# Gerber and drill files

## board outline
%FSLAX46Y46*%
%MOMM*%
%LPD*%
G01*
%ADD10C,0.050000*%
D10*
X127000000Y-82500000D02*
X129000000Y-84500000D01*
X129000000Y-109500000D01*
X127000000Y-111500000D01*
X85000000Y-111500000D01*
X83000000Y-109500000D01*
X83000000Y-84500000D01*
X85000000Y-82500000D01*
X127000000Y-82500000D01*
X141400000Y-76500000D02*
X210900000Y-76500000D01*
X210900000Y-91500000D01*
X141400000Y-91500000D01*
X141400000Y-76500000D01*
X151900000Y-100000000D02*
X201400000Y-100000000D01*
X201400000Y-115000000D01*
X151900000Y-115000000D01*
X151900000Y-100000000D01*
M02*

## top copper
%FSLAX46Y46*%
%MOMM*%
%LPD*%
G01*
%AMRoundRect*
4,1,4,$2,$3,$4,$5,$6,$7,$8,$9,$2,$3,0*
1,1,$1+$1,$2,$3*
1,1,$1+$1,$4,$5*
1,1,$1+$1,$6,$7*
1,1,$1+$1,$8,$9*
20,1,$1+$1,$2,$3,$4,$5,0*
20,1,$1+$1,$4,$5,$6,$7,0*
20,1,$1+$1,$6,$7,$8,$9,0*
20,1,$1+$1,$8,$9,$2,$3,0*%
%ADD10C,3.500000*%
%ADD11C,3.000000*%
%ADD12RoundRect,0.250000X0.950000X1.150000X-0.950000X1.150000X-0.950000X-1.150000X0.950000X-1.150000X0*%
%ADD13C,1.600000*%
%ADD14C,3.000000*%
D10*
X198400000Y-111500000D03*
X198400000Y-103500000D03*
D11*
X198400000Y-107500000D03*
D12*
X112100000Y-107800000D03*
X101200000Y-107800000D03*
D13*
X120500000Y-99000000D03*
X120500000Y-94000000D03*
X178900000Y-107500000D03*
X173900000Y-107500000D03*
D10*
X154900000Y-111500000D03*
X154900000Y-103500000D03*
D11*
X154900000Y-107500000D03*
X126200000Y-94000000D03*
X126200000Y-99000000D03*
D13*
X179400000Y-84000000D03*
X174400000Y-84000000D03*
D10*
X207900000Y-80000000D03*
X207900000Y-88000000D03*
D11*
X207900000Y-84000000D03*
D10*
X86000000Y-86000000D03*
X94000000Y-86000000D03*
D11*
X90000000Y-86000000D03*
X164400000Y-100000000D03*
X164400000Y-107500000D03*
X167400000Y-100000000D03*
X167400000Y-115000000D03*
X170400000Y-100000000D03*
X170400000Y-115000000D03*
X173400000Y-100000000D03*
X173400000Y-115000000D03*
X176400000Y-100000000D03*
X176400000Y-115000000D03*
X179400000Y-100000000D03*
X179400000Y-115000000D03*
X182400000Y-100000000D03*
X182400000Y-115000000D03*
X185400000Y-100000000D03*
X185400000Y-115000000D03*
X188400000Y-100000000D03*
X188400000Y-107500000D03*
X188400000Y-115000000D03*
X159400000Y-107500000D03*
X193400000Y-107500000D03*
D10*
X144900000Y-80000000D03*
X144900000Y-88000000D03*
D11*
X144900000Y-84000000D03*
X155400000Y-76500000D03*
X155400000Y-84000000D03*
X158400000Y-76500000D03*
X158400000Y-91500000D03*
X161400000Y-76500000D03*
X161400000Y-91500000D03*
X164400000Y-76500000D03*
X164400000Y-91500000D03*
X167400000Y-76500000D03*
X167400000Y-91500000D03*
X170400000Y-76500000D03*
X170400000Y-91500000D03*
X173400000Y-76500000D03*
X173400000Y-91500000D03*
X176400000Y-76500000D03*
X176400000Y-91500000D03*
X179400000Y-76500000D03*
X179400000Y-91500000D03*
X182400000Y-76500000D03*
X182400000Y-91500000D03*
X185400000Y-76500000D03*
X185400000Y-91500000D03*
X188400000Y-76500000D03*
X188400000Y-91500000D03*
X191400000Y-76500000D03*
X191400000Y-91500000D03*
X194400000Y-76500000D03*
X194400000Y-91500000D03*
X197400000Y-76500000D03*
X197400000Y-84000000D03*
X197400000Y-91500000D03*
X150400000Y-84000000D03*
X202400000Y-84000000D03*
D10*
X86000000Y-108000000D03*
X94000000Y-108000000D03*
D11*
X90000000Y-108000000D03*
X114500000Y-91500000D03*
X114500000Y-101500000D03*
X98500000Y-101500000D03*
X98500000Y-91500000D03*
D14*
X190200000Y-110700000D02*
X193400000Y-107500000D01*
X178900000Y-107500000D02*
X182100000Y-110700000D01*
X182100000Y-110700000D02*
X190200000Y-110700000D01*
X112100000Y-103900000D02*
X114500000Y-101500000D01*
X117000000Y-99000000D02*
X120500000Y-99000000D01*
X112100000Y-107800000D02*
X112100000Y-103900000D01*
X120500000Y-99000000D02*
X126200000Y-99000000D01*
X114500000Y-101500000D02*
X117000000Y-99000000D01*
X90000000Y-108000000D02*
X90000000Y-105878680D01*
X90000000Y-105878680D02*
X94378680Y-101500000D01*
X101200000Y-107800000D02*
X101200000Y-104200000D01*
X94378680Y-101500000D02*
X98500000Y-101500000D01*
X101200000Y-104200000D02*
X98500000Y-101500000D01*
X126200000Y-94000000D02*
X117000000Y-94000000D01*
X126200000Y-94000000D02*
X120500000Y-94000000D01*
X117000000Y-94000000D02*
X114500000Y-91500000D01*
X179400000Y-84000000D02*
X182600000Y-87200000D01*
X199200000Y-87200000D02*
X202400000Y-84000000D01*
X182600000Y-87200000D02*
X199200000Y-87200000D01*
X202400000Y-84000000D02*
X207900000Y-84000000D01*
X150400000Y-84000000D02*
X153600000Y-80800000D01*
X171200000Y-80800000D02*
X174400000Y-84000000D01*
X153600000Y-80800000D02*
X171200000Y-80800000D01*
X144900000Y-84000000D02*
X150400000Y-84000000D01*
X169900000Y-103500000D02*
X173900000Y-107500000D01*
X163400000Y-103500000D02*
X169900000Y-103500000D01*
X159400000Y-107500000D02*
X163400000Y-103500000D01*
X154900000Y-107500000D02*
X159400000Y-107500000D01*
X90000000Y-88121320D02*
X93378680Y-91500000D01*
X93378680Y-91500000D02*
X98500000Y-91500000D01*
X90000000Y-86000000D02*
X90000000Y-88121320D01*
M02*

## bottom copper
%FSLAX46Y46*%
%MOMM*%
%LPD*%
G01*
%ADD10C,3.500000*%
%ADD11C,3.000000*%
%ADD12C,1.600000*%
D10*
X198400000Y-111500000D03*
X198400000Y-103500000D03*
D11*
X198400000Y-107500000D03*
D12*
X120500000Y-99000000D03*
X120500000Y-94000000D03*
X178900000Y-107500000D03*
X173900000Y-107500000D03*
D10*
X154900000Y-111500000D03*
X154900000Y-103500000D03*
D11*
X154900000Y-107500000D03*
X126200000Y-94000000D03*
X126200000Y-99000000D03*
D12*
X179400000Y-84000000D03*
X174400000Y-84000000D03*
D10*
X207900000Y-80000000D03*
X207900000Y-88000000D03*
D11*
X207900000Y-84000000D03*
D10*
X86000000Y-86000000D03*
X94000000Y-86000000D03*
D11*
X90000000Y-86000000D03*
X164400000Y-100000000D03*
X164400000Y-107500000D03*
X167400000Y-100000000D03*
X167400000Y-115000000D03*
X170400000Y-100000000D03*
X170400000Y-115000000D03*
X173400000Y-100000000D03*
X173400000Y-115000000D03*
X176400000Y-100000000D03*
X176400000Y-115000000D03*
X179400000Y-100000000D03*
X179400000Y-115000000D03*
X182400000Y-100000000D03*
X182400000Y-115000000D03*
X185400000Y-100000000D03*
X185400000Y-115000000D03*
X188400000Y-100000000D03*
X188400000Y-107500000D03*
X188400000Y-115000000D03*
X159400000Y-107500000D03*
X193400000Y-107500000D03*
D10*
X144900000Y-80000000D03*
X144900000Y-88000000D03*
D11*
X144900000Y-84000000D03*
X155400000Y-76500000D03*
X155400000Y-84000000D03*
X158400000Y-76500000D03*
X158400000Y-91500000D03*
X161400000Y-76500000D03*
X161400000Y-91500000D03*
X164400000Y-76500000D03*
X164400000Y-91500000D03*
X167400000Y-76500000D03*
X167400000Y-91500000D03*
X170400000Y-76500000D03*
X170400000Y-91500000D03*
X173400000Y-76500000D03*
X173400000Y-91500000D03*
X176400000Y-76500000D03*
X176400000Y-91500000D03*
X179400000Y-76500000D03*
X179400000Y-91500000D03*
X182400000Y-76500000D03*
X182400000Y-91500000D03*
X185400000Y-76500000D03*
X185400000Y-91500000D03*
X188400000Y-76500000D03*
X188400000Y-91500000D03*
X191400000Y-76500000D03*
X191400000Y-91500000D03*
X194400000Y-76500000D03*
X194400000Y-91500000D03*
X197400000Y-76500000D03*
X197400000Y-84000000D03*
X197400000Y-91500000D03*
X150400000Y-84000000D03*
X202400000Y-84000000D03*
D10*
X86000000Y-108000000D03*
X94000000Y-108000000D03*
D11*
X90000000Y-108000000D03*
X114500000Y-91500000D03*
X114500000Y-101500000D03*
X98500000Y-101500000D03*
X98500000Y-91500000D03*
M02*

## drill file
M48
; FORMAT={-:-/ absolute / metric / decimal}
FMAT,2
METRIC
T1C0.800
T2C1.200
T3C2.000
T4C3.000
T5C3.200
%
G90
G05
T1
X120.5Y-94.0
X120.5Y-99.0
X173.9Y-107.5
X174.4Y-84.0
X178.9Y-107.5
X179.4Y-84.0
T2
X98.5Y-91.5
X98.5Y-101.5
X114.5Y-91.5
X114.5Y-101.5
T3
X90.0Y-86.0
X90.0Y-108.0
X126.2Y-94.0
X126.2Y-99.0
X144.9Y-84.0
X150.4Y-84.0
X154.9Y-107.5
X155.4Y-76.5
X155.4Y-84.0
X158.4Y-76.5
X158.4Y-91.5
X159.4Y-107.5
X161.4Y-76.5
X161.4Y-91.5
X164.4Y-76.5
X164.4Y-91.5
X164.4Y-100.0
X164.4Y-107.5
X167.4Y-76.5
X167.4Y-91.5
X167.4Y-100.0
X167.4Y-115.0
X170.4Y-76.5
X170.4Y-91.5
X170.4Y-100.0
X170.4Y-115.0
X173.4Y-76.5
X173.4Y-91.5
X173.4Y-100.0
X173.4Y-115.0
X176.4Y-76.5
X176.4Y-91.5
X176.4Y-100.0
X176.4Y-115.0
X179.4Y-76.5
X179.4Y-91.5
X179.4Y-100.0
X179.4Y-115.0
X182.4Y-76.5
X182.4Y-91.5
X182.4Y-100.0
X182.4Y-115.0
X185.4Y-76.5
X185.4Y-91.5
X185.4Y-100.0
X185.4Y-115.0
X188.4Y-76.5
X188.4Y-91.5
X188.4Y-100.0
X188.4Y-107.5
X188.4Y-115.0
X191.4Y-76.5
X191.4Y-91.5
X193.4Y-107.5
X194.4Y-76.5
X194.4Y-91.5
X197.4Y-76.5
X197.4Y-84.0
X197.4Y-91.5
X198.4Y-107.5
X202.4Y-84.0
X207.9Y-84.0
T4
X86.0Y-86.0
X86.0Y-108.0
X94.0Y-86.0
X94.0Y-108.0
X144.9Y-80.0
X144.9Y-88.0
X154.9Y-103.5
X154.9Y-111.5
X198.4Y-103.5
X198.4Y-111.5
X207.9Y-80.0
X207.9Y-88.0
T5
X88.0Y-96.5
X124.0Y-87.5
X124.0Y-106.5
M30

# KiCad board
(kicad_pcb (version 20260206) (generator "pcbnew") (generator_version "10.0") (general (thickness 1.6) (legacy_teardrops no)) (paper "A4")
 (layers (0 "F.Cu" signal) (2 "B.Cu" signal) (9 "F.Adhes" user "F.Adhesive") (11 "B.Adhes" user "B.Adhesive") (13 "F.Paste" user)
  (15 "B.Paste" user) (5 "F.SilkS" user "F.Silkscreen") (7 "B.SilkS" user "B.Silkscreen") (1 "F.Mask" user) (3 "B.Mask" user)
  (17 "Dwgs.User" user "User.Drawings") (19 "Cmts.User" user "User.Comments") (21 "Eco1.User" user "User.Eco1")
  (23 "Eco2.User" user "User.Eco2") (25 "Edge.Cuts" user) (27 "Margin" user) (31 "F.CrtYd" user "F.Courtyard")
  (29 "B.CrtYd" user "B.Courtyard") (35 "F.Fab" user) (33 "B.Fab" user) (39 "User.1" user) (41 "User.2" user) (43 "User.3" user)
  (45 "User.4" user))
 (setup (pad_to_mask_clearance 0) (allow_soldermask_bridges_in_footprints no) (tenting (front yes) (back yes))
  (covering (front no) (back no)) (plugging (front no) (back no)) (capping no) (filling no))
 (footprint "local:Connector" (layer "F.Cu") (at 198.4 107.5 180)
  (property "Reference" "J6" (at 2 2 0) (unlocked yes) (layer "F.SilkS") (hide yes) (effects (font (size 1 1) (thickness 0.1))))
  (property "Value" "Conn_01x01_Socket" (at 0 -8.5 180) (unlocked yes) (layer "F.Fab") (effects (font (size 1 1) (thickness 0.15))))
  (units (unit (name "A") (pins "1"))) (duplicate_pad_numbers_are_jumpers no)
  (pad "" thru_hole circle (at 0 -4 190) (size 3.5 3.5) (drill 3) (layers "*.Cu" "*.Mask") (remove_unused_layers no))
  (pad "" thru_hole circle (at 0 4 190) (size 3.5 3.5) (drill 3) (layers "*.Cu" "*.Mask") (remove_unused_layers no))
  (pad "1" thru_hole circle (at 0 0 190) (size 3 3) (drill 2) (layers "*.Cu" "*.Mask") (remove_unused_layers no) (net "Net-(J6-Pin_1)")))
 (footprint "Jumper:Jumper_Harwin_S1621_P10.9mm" (layer "F.Cu") (at 106.65 107.8 180)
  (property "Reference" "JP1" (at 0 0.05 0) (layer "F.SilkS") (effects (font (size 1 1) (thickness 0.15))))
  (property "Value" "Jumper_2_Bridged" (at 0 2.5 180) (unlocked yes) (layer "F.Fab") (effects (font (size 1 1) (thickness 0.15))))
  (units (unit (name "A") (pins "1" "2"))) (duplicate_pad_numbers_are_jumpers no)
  (pad "1" smd roundrect (at -5.45 0 180) (size 2.4 2.8) (layers "F.Cu" "F.Mask" "F.Paste") (roundrect_rratio 0.1041666667)
   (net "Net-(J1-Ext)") (thermal_bridge_angle 45))
  (pad "2" smd roundrect (at 5.45 0 180) (size 2.4 2.8) (layers "F.Cu" "F.Mask" "F.Paste") (roundrect_rratio 0.1041666667)
   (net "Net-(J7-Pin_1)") (thermal_bridge_angle 45)))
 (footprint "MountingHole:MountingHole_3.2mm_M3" (layer "F.Cu") (at 124 106.5)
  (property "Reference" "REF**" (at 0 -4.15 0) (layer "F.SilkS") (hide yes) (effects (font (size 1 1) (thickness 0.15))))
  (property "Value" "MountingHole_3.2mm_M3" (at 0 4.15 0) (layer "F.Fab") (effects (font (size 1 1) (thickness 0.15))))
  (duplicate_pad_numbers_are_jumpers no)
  (pad "" np_thru_hole circle (at 0 0) (size 3.2 3.2) (drill 3.2) (layers "*.Cu" "*.Mask")))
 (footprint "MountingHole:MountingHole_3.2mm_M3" (layer "F.Cu") (at 88 96.5)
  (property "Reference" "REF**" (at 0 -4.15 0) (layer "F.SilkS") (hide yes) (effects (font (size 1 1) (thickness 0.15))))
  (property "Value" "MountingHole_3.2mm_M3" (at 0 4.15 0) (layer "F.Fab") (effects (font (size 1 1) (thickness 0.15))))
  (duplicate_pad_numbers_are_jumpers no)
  (pad "" np_thru_hole circle (at 0 0) (size 3.2 3.2) (drill 3.2) (layers "*.Cu" "*.Mask")))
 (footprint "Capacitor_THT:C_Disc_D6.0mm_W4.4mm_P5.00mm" (layer "F.Cu") (at 120.5 99 90)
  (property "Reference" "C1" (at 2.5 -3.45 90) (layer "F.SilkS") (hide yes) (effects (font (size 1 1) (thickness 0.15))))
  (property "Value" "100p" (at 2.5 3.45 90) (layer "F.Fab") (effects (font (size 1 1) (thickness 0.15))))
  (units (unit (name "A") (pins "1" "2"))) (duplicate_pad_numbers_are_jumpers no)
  (pad "1" thru_hole circle (at 0 0 90) (size 1.6 1.6) (drill 0.8) (layers "*.Cu" "*.Mask") (remove_unused_layers no) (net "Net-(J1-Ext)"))
  (pad "2" thru_hole circle (at 5 0 90) (size 1.6 1.6) (drill 0.8) (layers "*.Cu" "*.Mask") (remove_unused_layers no) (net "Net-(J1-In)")))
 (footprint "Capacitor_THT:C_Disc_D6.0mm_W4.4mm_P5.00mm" (layer "F.Cu") (at 178.9 107.5 180)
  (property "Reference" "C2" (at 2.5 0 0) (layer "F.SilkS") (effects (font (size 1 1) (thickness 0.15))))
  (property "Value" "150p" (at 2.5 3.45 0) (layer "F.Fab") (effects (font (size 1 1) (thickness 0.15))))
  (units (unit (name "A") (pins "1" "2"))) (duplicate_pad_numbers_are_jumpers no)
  (pad "1" thru_hole circle (at 0 0 180) (size 1.6 1.6) (drill 0.8) (layers "*.Cu" "*.Mask") (remove_unused_layers no)
   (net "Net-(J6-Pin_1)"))
  (pad "2" thru_hole circle (at 5 0 180) (size 1.6 1.6) (drill 0.8) (layers "*.Cu" "*.Mask") (remove_unused_layers no)
   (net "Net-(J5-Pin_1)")))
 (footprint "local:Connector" (layer "F.Cu") (at 154.9 107.5 180)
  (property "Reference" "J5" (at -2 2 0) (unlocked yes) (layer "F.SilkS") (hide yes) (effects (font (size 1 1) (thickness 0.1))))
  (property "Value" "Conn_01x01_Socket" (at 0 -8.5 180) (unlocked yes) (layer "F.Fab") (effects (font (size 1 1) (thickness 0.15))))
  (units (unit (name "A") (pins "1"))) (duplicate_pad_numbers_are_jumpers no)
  (pad "" thru_hole circle (at 0 -4 190) (size 3.5 3.5) (drill 3) (layers "*.Cu" "*.Mask") (remove_unused_layers no))
  (pad "" thru_hole circle (at 0 4 190) (size 3.5 3.5) (drill 3) (layers "*.Cu" "*.Mask") (remove_unused_layers no))
  (pad "1" thru_hole circle (at 0 0 190) (size 3 3) (drill 2) (layers "*.Cu" "*.Mask") (remove_unused_layers no) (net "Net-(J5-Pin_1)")))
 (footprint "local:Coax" (layer "F.Cu") (at 126.2 96)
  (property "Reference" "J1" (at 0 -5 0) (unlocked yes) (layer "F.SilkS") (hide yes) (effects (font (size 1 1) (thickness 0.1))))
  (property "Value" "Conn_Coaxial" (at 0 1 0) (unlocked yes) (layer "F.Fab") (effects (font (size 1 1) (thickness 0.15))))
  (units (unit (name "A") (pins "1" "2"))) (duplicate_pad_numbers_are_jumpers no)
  (pad "1" thru_hole circle (at 0 -2 10) (size 3 3) (drill 2) (layers "*.Cu" "*.Mask") (remove_unused_layers no) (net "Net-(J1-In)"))
  (pad "2" thru_hole circle (at 0 3 10) (size 3 3) (drill 2) (layers "*.Cu" "*.Mask") (remove_unused_layers no) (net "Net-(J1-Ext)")))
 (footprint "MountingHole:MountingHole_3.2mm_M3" (layer "F.Cu") (at 124 87.5)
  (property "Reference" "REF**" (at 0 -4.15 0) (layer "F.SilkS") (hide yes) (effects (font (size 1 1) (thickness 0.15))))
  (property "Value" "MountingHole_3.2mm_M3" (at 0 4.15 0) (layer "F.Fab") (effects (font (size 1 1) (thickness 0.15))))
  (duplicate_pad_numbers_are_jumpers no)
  (pad "" np_thru_hole circle (at 0 0) (size 3.2 3.2) (drill 3.2) (layers "*.Cu" "*.Mask")))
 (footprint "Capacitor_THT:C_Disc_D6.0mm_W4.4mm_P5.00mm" (layer "F.Cu") (at 179.4 84 180)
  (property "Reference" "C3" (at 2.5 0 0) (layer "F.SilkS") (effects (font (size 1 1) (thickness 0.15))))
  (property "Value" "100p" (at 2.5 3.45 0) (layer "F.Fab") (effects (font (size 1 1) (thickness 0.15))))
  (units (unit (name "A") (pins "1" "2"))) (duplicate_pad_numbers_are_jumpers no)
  (pad "1" thru_hole circle (at 0 0 180) (size 1.6 1.6) (drill 0.8) (layers "*.Cu" "*.Mask") (remove_unused_layers no)
   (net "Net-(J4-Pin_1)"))
  (pad "2" thru_hole circle (at 5 0 180) (size 1.6 1.6) (drill 0.8) (layers "*.Cu" "*.Mask") (remove_unused_layers no)
   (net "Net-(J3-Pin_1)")))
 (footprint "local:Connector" (layer "F.Cu") (at 207.9 84)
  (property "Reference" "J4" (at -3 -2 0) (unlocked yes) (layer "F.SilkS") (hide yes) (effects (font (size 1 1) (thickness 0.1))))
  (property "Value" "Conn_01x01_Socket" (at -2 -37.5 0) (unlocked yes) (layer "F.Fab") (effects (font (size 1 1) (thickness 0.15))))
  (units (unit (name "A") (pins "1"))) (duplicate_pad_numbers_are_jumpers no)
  (pad "" thru_hole circle (at 0 -4 10) (size 3.5 3.5) (drill 3) (layers "*.Cu" "*.Mask") (remove_unused_layers no))
  (pad "" thru_hole circle (at 0 4 10) (size 3.5 3.5) (drill 3) (layers "*.Cu" "*.Mask") (remove_unused_layers no))
  (pad "1" thru_hole circle (at 0 0 10) (size 3 3) (drill 2) (layers "*.Cu" "*.Mask") (remove_unused_layers no) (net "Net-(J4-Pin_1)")))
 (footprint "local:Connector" (layer "F.Cu") (at 90 86 90)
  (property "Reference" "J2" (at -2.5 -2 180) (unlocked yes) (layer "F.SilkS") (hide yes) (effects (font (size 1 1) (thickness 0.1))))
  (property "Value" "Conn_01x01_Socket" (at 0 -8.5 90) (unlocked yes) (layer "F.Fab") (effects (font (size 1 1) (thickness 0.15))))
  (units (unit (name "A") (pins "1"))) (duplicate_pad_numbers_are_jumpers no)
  (pad "" thru_hole circle (at 0 -4 100) (size 3.5 3.5) (drill 3) (layers "*.Cu" "*.Mask") (remove_unused_layers no))
  (pad "" thru_hole circle (at 0 4 100) (size 3.5 3.5) (drill 3) (layers "*.Cu" "*.Mask") (remove_unused_layers no))
  (pad "1" thru_hole circle (at 0 0 100) (size 3 3) (drill 2) (layers "*.Cu" "*.Mask") (remove_unused_layers no) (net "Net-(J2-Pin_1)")))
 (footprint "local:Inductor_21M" (layer "F.Cu") (at 167.4 107)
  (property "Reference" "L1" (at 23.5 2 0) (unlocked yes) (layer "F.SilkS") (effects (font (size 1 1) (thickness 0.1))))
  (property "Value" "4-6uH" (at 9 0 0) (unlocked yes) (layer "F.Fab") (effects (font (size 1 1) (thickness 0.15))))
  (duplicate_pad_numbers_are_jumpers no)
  (pad "" thru_hole circle (at -3 -7 10) (size 3 3) (drill 2) (layers "*.Cu" "*.Mask") (remove_unused_layers no))
  (pad "" thru_hole circle (at -3 0.5 10) (size 3 3) (drill 2) (layers "*.Cu" "*.Mask") (remove_unused_layers no))
  (pad "" thru_hole circle (at 0 -7 10) (size 3 3) (drill 2) (layers "*.Cu" "*.Mask") (remove_unused_layers no))
  (pad "" thru_hole circle (at 0 8 10) (size 3 3) (drill 2) (layers "*.Cu" "*.Mask") (remove_unused_layers no))
  (pad "" thru_hole circle (at 3 -7 10) (size 3 3) (drill 2) (layers "*.Cu" "*.Mask") (remove_unused_layers no))
  (pad "" thru_hole circle (at 3 8 10) (size 3 3) (drill 2) (layers "*.Cu" "*.Mask") (remove_unused_layers no))
  (pad "" thru_hole circle (at 6 -7 10) (size 3 3) (drill 2) (layers "*.Cu" "*.Mask") (remove_unused_layers no))
  (pad "" thru_hole circle (at 6 8 10) (size 3 3) (drill 2) (layers "*.Cu" "*.Mask") (remove_unused_layers no))
  (pad "" thru_hole circle (at 9 -7 10) (size 3 3) (drill 2) (layers "*.Cu" "*.Mask") (remove_unused_layers no))
  (pad "" thru_hole circle (at 9 8 10) (size 3 3) (drill 2) (layers "*.Cu" "*.Mask") (remove_unused_layers no))
  (pad "" thru_hole circle (at 12 -7 10) (size 3 3) (drill 2) (layers "*.Cu" "*.Mask") (remove_unused_layers no))
  (pad "" thru_hole circle (at 12 8 10) (size 3 3) (drill 2) (layers "*.Cu" "*.Mask") (remove_unused_layers no))
  (pad "" thru_hole circle (at 15 -7 10) (size 3 3) (drill 2) (layers "*.Cu" "*.Mask") (remove_unused_layers no))
  (pad "" thru_hole circle (at 15 8 10) (size 3 3) (drill 2) (layers "*.Cu" "*.Mask") (remove_unused_layers no))
  (pad "" thru_hole circle (at 18 -7 10) (size 3 3) (drill 2) (layers "*.Cu" "*.Mask") (remove_unused_layers no))
  (pad "" thru_hole circle (at 18 8 10) (size 3 3) (drill 2) (layers "*.Cu" "*.Mask") (remove_unused_layers no))
  (pad "" thru_hole circle (at 21 -7 10) (size 3 3) (drill 2) (layers "*.Cu" "*.Mask") (remove_unused_layers no))
  (pad "" thru_hole circle (at 21 0.5 10) (size 3 3) (drill 2) (layers "*.Cu" "*.Mask") (remove_unused_layers no))
  (pad "" thru_hole circle (at 21 8 10) (size 3 3) (drill 2) (layers "*.Cu" "*.Mask") (remove_unused_layers no))
  (pad "1" thru_hole circle (at -8 0.5 10) (size 3 3) (drill 2) (layers "*.Cu" "*.Mask") (remove_unused_layers no) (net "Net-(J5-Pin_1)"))
  (pad "2" thru_hole circle (at 26 0.5 10) (size 3 3) (drill 2) (layers "*.Cu" "*.Mask") (remove_unused_layers no) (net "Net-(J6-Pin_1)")))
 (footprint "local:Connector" (layer "F.Cu") (at 144.9 84)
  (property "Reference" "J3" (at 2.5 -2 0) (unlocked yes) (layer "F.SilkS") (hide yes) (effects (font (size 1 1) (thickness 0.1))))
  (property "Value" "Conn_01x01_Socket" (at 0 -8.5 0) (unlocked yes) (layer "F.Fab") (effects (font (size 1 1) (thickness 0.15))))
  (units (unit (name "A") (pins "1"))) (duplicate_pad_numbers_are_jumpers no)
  (pad "" thru_hole circle (at 0 -4 10) (size 3.5 3.5) (drill 3) (layers "*.Cu" "*.Mask") (remove_unused_layers no))
  (pad "" thru_hole circle (at 0 4 10) (size 3.5 3.5) (drill 3) (layers "*.Cu" "*.Mask") (remove_unused_layers no))
  (pad "1" thru_hole circle (at 0 0 10) (size 3 3) (drill 2) (layers "*.Cu" "*.Mask") (remove_unused_layers no) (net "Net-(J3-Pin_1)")))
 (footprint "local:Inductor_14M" (layer "F.Cu") (at 176.4 83.5)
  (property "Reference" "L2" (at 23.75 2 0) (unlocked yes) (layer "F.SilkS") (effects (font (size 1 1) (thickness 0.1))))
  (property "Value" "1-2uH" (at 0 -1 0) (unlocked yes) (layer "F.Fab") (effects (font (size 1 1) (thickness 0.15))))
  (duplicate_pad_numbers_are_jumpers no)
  (pad "" thru_hole circle (at -21 -7 10) (size 3 3) (drill 2) (layers "*.Cu" "*.Mask") (remove_unused_layers no))
  (pad "" thru_hole circle (at -21 0.5 10) (size 3 3) (drill 2) (layers "*.Cu" "*.Mask") (remove_unused_layers no))
  (pad "" thru_hole circle (at -18 -7 10) (size 3 3) (drill 2) (layers "*.Cu" "*.Mask") (remove_unused_layers no))
  (pad "" thru_hole circle (at -18 8 10) (size 3 3) (drill 2) (layers "*.Cu" "*.Mask") (remove_unused_layers no))
  (pad "" thru_hole circle (at -15 -7 10) (size 3 3) (drill 2) (layers "*.Cu" "*.Mask") (remove_unused_layers no))
  (pad "" thru_hole circle (at -15 8 10) (size 3 3) (drill 2) (layers "*.Cu" "*.Mask") (remove_unused_layers no))
  (pad "" thru_hole circle (at -12 -7 10) (size 3 3) (drill 2) (layers "*.Cu" "*.Mask") (remove_unused_layers no))
  (pad "" thru_hole circle (at -12 8 10) (size 3 3) (drill 2) (layers "*.Cu" "*.Mask") (remove_unused_layers no))
  (pad "" thru_hole circle (at -9 -7 10) (size 3 3) (drill 2) (layers "*.Cu" "*.Mask") (remove_unused_layers no))
  (pad "" thru_hole circle (at -9 8 10) (size 3 3) (drill 2) (layers "*.Cu" "*.Mask") (remove_unused_layers no))
  (pad "" thru_hole circle (at -6 -7 10) (size 3 3) (drill 2) (layers "*.Cu" "*.Mask") (remove_unused_layers no))
  (pad "" thru_hole circle (at -6 8 10) (size 3 3) (drill 2) (layers "*.Cu" "*.Mask") (remove_unused_layers no))
  (pad "" thru_hole circle (at -3 -7 10) (size 3 3) (drill 2) (layers "*.Cu" "*.Mask") (remove_unused_layers no))
  (pad "" thru_hole circle (at -3 8 10) (size 3 3) (drill 2) (layers "*.Cu" "*.Mask") (remove_unused_layers no))
  (pad "" thru_hole circle (at 0 -7 10) (size 3 3) (drill 2) (layers "*.Cu" "*.Mask") (remove_unused_layers no))
  (pad "" thru_hole circle (at 0 8 10) (size 3 3) (drill 2) (layers "*.Cu" "*.Mask") (remove_unused_layers no))
  (pad "" thru_hole circle (at 3 -7 10) (size 3 3) (drill 2) (layers "*.Cu" "*.Mask") (remove_unused_layers no))
  (pad "" thru_hole circle (at 3 8 10) (size 3 3) (drill 2) (layers "*.Cu" "*.Mask") (remove_unused_layers no))
  (pad "" thru_hole circle (at 6 -7 10) (size 3 3) (drill 2) (layers "*.Cu" "*.Mask") (remove_unused_layers no))
  (pad "" thru_hole circle (at 6 8 10) (size 3 3) (drill 2) (layers "*.Cu" "*.Mask") (remove_unused_layers no))
  (pad "" thru_hole circle (at 9 -7 10) (size 3 3) (drill 2) (layers "*.Cu" "*.Mask") (remove_unused_layers no))
  (pad "" thru_hole circle (at 9 8 10) (size 3 3) (drill 2) (layers "*.Cu" "*.Mask") (remove_unused_layers no))
  (pad "" thru_hole circle (at 12 -7 10) (size 3 3) (drill 2) (layers "*.Cu" "*.Mask") (remove_unused_layers no))
  (pad "" thru_hole circle (at 12 8 10) (size 3 3) (drill 2) (layers "*.Cu" "*.Mask") (remove_unused_layers no))
  (pad "" thru_hole circle (at 15 -7 10) (size 3 3) (drill 2) (layers "*.Cu" "*.Mask") (remove_unused_layers no))
  (pad "" thru_hole circle (at 15 8 10) (size 3 3) (drill 2) (layers "*.Cu" "*.Mask") (remove_unused_layers no))
  (pad "" thru_hole circle (at 18 -7 10) (size 3 3) (drill 2) (layers "*.Cu" "*.Mask") (remove_unused_layers no))
  (pad "" thru_hole circle (at 18 8 10) (size 3 3) (drill 2) (layers "*.Cu" "*.Mask") (remove_unused_layers no))
  (pad "" thru_hole circle (at 21 -7 10) (size 3 3) (drill 2) (layers "*.Cu" "*.Mask") (remove_unused_layers no))
  (pad "" thru_hole circle (at 21 0.5 10) (size 3 3) (drill 2) (layers "*.Cu" "*.Mask") (remove_unused_layers no))
  (pad "" thru_hole circle (at 21 8 10) (size 3 3) (drill 2) (layers "*.Cu" "*.Mask") (remove_unused_layers no))
  (pad "1" thru_hole circle (at -26 0.5 10) (size 3 3) (drill 2) (layers "*.Cu" "*.Mask") (remove_unused_layers no) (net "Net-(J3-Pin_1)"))
  (pad "2" thru_hole circle (at 26 0.5 10) (size 3 3) (drill 2) (layers "*.Cu" "*.Mask") (remove_unused_layers no) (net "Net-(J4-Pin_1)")))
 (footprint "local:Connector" (layer "F.Cu") (at 90 108 90)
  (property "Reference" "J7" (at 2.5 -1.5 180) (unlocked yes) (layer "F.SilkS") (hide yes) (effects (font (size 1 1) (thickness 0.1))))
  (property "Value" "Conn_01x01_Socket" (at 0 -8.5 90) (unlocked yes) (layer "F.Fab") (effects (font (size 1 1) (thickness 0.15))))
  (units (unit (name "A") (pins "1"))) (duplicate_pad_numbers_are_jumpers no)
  (pad "" thru_hole circle (at 0 -4 100) (size 3.5 3.5) (drill 3) (layers "*.Cu" "*.Mask") (remove_unused_layers no))
  (pad "" thru_hole circle (at 0 4 100) (size 3.5 3.5) (drill 3) (layers "*.Cu" "*.Mask") (remove_unused_layers no))
  (pad "1" thru_hole circle (at 0 0 100) (size 3 3) (drill 2) (layers "*.Cu" "*.Mask") (remove_unused_layers no) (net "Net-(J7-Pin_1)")))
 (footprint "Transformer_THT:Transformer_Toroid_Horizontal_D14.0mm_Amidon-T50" (layer "F.Cu") (at 114.5 91.5 180)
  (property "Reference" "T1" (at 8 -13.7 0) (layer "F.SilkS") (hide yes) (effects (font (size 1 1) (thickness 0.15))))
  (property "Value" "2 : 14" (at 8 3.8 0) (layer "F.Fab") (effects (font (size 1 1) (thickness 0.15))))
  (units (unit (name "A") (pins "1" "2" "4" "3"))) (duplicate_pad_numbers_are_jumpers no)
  (pad "1" thru_hole circle (at 0 0 180) (size 3 3) (drill 1.2) (layers "*.Cu" "*.Mask") (remove_unused_layers no) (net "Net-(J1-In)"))
  (pad "2" thru_hole circle (at 0 -10 180) (size 3 3) (drill 1.2) (layers "*.Cu" "*.Mask") (remove_unused_layers no) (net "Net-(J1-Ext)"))
  (pad "3" thru_hole circle (at 16 -10 180) (size 3 3) (drill 1.2) (layers "*.Cu" "*.Mask") (remove_unused_layers no) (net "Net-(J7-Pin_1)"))
  (pad "4" thru_hole circle (at 16 0 180) (size 3 3) (drill 1.2) (layers "*.Cu" "*.Mask") (remove_unused_layers no) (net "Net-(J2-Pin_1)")))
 (gr_poly
  (pts (xy 127 82.5) (xy 129 84.5) (xy 129 109.5) (xy 127 111.5) (xy 85 111.5) (xy 83 109.5) (xy 83 84.5) (xy 85 82.5))
  (stroke (width 0.05) (type solid)) (fill no) (layer "Edge.Cuts"))
 (gr_rect (start 141.4 76.5) (end 210.9 91.5) (stroke (width 0.05) (type default)) (fill no) (layer "Edge.Cuts"))
 (gr_rect (start 151.9 100) (end 201.4 115) (stroke (width 0.05) (type default)) (fill no) (layer "Edge.Cuts"))
 (segment (start 190.2 110.7) (end 193.4 107.5) (width 3) (layer "F.Cu") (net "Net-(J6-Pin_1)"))
 (segment (start 178.9 107.5) (end 182.1 110.7) (width 3) (layer "F.Cu") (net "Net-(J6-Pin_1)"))
 (segment (start 182.1 110.7) (end 190.2 110.7) (width 3) (layer "F.Cu") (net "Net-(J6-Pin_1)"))
 (segment (start 112.1 103.9) (end 114.5 101.5) (width 3) (layer "F.Cu") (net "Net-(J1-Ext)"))
 (segment (start 117 99) (end 120.5 99) (width 3) (layer "F.Cu") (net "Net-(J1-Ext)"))
 (segment (start 112.1 107.8) (end 112.1 103.9) (width 3) (layer "F.Cu") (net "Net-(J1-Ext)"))
 (segment (start 120.5 99) (end 126.2 99) (width 3) (layer "F.Cu") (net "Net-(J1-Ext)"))
 (segment (start 114.5 101.5) (end 117 99) (width 3) (layer "F.Cu") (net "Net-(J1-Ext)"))
 (segment (start 90 108) (end 90 105.87868) (width 3) (layer "F.Cu") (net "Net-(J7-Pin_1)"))
 (segment (start 90 105.87868) (end 94.37868 101.5) (width 3) (layer "F.Cu") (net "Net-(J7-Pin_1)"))
 (segment (start 101.2 107.8) (end 101.2 104.2) (width 3) (layer "F.Cu") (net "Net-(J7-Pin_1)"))
 (segment (start 94.37868 101.5) (end 98.5 101.5) (width 3) (layer "F.Cu") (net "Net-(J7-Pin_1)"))
 (segment (start 101.2 104.2) (end 98.5 101.5) (width 3) (layer "F.Cu") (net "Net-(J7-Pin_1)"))
 (segment (start 126.2 94) (end 117 94) (width 3) (layer "F.Cu") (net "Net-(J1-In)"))
 (segment (start 126.2 94) (end 120.5 94) (width 3) (layer "F.Cu") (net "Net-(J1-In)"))
 (segment (start 117 94) (end 114.5 91.5) (width 3) (layer "F.Cu") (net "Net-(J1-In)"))
 (segment (start 179.4 84) (end 182.6 87.2) (width 3) (layer "F.Cu") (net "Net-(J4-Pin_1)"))
 (segment (start 199.2 87.2) (end 202.4 84) (width 3) (layer "F.Cu") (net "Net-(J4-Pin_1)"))
 (segment (start 182.6 87.2) (end 199.2 87.2) (width 3) (layer "F.Cu") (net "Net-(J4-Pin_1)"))
 (segment (start 202.4 84) (end 207.9 84) (width 3) (layer "F.Cu") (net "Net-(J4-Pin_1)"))
 (segment (start 150.4 84) (end 153.6 80.8) (width 3) (layer "F.Cu") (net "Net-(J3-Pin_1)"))
 (segment (start 171.2 80.8) (end 174.4 84) (width 3) (layer "F.Cu") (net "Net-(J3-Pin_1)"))
 (segment (start 153.6 80.8) (end 171.2 80.8) (width 3) (layer "F.Cu") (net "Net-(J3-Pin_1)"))
 (segment (start 144.9 84) (end 150.4 84) (width 3) (layer "F.Cu") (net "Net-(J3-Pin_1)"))
 (segment (start 169.9 103.5) (end 173.9 107.5) (width 3) (layer "F.Cu") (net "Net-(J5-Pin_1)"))
 (segment (start 163.4 103.5) (end 169.9 103.5) (width 3) (layer "F.Cu") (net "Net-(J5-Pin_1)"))
 (segment (start 159.4 107.5) (end 163.4 103.5) (width 3) (layer "F.Cu") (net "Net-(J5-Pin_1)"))
 (segment (start 154.9 107.5) (end 159.4 107.5) (width 3) (layer "F.Cu") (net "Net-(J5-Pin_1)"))
 (segment (start 90 88.12132) (end 93.37868 91.5) (width 3) (layer "F.Cu") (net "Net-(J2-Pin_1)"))
 (segment (start 93.37868 91.5) (end 98.5 91.5) (width 3) (layer "F.Cu") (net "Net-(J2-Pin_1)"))
 (segment (start 90 86) (end 90 88.12132) (width 3) (layer "F.Cu") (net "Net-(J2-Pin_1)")))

